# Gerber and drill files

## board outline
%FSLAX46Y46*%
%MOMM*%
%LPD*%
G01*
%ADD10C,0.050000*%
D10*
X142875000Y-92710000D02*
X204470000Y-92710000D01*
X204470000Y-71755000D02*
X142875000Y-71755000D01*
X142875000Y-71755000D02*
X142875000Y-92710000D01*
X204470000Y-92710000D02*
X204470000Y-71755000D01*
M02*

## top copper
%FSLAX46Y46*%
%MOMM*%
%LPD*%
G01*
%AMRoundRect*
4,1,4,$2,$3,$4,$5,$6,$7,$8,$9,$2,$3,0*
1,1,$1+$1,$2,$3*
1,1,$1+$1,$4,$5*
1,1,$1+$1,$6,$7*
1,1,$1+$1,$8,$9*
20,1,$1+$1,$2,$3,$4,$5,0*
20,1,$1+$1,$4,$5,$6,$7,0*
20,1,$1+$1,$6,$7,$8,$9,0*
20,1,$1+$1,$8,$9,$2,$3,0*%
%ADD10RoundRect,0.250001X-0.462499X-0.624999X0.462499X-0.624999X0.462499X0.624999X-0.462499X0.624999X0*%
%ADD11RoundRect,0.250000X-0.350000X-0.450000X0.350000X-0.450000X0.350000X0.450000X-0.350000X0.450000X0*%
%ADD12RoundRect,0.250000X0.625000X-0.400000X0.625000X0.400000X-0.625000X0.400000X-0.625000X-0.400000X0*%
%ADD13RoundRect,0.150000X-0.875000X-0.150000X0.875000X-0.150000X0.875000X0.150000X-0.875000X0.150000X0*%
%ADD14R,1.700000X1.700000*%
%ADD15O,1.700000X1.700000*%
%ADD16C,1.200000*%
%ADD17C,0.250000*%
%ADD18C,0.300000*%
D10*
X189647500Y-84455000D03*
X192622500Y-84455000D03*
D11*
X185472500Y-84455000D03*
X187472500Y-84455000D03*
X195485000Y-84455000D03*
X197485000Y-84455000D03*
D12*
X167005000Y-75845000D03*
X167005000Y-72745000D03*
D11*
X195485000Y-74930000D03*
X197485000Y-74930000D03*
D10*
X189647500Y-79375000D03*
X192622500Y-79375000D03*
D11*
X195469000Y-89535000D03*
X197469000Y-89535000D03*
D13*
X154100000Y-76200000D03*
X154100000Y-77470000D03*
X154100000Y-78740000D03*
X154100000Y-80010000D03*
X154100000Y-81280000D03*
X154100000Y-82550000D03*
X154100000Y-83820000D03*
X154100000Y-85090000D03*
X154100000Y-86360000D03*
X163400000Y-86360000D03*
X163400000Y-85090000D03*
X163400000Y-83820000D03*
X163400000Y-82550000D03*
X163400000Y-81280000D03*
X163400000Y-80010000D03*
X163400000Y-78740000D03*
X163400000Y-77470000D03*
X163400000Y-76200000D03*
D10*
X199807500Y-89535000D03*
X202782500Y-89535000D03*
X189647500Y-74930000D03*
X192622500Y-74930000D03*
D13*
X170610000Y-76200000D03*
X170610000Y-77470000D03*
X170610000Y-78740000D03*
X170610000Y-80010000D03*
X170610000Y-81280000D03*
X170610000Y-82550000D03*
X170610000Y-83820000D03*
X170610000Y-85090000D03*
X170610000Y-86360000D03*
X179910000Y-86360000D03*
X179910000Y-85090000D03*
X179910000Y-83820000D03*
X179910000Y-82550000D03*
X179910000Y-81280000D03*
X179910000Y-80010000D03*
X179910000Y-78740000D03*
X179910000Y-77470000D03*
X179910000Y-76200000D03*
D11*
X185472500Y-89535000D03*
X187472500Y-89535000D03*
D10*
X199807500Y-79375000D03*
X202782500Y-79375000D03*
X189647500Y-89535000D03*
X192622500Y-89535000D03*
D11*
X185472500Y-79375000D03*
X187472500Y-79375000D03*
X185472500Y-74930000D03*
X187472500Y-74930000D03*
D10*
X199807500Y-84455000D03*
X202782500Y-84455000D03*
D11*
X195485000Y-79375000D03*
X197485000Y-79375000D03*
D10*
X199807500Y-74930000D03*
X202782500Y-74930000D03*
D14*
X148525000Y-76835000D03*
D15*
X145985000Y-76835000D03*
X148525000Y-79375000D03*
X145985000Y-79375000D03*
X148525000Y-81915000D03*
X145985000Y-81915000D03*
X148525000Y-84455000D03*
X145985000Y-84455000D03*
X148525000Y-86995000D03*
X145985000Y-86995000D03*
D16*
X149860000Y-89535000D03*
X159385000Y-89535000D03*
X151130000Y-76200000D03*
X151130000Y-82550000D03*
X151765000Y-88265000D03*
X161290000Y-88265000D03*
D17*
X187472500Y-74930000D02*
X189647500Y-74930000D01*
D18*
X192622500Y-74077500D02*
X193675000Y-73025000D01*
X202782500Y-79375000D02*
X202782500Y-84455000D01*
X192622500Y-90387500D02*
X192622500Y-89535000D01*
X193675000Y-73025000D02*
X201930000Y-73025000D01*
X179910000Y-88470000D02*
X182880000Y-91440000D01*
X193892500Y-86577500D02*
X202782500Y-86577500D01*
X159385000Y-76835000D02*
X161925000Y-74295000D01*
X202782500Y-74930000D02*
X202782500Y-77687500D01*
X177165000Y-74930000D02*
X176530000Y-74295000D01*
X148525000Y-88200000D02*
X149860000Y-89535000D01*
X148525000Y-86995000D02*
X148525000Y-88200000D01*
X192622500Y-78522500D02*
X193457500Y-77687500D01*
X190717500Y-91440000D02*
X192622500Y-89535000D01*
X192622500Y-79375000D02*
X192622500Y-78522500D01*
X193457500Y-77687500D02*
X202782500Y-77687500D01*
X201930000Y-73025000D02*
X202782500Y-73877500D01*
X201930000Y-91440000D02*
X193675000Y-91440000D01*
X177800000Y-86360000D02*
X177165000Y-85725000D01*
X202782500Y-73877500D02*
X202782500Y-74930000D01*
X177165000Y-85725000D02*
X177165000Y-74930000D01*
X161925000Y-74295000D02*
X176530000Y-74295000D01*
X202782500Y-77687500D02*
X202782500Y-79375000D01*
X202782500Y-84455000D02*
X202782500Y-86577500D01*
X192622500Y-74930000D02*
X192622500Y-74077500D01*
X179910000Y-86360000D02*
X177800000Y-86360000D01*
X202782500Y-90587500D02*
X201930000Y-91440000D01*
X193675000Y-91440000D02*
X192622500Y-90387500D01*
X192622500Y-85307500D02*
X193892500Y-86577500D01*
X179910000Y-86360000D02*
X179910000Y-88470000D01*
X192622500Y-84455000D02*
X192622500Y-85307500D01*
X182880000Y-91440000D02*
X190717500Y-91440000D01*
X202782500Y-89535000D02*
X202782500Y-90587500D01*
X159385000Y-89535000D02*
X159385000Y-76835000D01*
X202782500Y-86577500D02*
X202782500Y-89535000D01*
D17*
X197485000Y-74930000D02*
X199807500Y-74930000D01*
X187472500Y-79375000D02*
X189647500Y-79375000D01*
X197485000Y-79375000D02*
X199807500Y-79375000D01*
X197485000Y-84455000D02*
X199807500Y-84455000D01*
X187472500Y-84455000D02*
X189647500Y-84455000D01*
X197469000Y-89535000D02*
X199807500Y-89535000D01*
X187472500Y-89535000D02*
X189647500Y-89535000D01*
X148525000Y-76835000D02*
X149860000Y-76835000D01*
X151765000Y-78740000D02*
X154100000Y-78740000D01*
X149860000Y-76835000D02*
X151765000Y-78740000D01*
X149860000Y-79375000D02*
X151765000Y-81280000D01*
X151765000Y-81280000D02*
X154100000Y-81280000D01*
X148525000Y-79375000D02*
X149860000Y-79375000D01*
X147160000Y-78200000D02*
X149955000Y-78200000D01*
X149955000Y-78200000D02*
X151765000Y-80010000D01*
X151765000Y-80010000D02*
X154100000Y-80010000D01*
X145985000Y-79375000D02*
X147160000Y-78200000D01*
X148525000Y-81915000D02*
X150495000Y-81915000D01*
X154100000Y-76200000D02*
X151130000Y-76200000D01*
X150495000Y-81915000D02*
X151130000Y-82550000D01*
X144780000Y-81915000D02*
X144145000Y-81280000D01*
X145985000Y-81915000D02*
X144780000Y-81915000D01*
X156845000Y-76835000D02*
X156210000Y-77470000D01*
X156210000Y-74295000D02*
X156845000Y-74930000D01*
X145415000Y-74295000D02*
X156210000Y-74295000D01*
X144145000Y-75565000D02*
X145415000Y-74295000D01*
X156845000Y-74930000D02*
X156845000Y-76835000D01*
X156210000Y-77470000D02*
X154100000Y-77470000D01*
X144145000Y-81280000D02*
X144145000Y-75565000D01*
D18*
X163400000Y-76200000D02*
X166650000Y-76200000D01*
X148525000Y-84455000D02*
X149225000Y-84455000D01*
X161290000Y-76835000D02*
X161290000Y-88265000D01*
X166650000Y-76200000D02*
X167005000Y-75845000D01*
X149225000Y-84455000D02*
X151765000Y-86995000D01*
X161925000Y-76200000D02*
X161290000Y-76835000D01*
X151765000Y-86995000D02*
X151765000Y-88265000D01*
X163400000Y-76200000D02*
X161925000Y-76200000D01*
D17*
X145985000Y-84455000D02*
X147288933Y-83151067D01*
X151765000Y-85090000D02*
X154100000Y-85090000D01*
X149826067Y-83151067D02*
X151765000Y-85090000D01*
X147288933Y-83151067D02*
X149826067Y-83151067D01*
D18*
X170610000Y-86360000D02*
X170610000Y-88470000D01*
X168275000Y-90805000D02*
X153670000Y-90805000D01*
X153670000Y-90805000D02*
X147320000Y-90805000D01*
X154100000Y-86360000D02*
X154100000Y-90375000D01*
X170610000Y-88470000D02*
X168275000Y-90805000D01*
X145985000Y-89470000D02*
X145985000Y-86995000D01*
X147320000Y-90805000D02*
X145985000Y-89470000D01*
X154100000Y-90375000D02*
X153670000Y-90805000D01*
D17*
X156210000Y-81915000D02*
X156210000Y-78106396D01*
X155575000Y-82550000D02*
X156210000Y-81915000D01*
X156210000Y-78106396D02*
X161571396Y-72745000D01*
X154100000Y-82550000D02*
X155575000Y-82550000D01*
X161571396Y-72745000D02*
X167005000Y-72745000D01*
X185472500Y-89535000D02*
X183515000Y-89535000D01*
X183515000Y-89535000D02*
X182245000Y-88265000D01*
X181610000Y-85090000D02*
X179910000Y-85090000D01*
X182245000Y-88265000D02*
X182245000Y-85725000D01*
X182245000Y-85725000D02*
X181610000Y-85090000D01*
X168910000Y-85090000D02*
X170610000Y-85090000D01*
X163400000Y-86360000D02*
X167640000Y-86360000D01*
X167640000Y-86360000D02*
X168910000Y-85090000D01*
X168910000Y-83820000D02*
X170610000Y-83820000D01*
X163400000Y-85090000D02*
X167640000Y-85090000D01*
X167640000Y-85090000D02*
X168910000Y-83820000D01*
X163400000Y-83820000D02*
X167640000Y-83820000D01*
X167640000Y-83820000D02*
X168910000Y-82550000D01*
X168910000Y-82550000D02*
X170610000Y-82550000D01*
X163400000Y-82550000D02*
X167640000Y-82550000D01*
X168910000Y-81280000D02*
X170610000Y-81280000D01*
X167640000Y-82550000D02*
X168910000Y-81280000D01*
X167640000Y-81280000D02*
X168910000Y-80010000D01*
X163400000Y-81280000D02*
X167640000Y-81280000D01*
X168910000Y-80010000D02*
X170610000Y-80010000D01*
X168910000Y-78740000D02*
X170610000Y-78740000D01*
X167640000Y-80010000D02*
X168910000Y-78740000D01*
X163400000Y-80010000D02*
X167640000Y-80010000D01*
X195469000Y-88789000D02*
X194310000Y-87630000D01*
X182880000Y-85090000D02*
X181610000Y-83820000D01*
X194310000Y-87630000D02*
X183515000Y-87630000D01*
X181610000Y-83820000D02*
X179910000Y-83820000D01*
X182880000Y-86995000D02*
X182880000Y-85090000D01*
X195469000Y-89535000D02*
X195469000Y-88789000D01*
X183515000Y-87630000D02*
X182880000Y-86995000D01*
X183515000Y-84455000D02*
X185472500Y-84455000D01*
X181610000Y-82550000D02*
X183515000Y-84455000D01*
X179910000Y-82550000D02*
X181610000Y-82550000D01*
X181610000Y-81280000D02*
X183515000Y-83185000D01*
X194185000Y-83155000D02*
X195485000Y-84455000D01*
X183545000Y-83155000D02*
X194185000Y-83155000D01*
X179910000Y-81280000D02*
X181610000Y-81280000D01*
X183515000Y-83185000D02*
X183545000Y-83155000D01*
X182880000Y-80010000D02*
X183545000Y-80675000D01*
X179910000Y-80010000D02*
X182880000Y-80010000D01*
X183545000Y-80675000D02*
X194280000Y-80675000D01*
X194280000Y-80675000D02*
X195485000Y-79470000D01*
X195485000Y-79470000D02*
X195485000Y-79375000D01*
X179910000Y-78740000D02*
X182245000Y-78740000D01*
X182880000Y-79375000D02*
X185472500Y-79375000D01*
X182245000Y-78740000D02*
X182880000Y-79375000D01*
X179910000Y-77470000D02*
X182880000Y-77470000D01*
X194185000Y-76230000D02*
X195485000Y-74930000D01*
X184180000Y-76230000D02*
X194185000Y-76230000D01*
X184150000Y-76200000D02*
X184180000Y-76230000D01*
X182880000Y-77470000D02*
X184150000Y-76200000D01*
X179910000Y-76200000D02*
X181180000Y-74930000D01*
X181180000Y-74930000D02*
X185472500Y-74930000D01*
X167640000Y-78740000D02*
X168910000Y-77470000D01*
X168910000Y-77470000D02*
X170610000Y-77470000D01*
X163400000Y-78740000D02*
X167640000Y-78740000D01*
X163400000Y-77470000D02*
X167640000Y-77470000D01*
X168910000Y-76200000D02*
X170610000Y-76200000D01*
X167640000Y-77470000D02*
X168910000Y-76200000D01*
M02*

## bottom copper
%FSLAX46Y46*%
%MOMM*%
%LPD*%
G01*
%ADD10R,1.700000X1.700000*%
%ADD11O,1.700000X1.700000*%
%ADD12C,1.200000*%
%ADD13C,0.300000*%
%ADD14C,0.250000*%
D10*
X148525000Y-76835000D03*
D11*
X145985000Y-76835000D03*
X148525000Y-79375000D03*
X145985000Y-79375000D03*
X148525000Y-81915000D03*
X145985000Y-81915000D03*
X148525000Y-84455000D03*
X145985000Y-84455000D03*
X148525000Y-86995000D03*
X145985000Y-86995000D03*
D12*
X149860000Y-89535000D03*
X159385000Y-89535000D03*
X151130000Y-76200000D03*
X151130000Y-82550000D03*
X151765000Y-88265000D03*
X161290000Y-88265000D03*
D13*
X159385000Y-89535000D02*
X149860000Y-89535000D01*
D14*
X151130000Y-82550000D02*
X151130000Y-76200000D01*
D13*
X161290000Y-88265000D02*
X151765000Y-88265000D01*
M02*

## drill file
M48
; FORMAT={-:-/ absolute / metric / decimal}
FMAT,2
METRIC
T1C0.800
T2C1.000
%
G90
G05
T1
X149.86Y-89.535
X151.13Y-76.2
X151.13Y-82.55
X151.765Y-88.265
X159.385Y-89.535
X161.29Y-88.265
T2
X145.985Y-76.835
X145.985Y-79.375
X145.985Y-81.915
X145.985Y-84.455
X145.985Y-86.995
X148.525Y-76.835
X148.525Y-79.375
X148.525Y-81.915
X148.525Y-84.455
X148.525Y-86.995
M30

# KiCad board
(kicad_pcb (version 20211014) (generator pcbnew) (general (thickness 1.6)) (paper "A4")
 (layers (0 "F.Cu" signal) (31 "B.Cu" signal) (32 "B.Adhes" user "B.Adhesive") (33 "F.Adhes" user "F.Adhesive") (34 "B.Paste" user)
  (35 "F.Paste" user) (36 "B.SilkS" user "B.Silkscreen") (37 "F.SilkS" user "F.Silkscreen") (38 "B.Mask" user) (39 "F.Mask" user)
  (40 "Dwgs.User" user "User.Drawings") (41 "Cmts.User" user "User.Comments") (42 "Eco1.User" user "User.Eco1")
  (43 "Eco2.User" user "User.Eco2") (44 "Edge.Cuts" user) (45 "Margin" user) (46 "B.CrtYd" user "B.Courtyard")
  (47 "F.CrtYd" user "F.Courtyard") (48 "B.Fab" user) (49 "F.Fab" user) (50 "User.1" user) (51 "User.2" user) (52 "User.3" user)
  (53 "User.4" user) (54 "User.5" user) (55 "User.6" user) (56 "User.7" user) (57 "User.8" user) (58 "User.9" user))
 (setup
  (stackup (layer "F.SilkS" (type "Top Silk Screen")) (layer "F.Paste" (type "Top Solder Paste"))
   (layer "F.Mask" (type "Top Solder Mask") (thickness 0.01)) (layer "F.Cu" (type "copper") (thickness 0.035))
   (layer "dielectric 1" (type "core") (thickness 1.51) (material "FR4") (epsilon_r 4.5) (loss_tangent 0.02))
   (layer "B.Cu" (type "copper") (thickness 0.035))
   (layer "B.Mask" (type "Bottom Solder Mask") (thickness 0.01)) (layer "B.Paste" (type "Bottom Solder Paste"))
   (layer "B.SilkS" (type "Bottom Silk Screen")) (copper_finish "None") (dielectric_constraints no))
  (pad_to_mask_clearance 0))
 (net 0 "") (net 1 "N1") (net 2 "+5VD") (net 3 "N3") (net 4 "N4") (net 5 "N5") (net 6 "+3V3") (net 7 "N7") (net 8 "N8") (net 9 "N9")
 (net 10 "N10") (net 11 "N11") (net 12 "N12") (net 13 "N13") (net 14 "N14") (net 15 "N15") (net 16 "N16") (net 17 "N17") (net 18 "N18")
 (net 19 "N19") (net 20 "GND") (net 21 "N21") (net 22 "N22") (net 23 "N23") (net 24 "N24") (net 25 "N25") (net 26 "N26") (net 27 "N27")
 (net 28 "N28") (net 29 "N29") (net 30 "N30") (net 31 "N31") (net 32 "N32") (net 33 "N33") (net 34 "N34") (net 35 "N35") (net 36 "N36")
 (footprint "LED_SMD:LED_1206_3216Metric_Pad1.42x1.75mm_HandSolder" (layer "F.Cu") (at 191.135 84.455)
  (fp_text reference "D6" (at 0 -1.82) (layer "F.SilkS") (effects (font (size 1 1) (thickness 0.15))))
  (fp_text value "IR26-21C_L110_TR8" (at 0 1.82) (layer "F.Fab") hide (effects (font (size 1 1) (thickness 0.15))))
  (pad "1" smd roundrect (at -1.4875 0) (size 1.425 1.75) (layers "F.Cu" "F.Paste" "F.Mask") (roundrect_rratio 0.175439) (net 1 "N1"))
  (pad "2" smd roundrect (at 1.4875 0) (size 1.425 1.75) (layers "F.Cu" "F.Paste" "F.Mask") (roundrect_rratio 0.175439) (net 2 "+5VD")))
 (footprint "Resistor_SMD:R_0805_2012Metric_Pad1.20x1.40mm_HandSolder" (layer "F.Cu") (at 186.4725 84.455)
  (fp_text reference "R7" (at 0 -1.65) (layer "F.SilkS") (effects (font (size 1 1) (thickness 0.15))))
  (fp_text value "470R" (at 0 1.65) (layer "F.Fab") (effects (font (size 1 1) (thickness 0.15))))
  (pad "1" smd roundrect (at -1 0) (size 1.2 1.4) (layers "F.Cu" "F.Paste" "F.Mask") (roundrect_rratio 0.208333) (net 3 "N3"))
  (pad "2" smd roundrect (at 1 0) (size 1.2 1.4) (layers "F.Cu" "F.Paste" "F.Mask") (roundrect_rratio 0.208333) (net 1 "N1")))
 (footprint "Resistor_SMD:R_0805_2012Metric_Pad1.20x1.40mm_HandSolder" (layer "F.Cu") (at 196.485 84.455)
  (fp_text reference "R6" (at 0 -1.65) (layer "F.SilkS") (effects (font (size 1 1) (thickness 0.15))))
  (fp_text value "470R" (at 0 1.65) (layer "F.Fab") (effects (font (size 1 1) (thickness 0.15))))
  (pad "1" smd roundrect (at -1 0) (size 1.2 1.4) (layers "F.Cu" "F.Paste" "F.Mask") (roundrect_rratio 0.208333) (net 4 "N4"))
  (pad "2" smd roundrect (at 1 0) (size 1.2 1.4) (layers "F.Cu" "F.Paste" "F.Mask") (roundrect_rratio 0.208333) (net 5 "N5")))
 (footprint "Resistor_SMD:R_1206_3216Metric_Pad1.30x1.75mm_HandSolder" (layer "F.Cu") (at 167.005 74.295 90)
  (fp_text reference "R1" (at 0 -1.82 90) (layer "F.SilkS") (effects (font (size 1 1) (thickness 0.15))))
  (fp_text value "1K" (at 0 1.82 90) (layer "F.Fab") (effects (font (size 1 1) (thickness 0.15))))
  (pad "1" smd roundrect (at -1.55 0 90) (size 1.3 1.75) (layers "F.Cu" "F.Paste" "F.Mask") (roundrect_rratio 0.192308) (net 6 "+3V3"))
  (pad "2" smd roundrect (at 1.55 0 90) (size 1.3 1.75) (layers "F.Cu" "F.Paste" "F.Mask") (roundrect_rratio 0.192308) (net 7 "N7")))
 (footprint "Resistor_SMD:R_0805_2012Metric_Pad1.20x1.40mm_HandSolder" (layer "F.Cu") (at 196.485 74.93)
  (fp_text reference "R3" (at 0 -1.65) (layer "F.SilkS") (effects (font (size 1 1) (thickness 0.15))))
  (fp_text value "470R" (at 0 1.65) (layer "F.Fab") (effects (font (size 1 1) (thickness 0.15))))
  (pad "1" smd roundrect (at -1 0) (size 1.2 1.4) (layers "F.Cu" "F.Paste" "F.Mask") (roundrect_rratio 0.208333) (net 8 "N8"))
  (pad "2" smd roundrect (at 1 0) (size 1.2 1.4) (layers "F.Cu" "F.Paste" "F.Mask") (roundrect_rratio 0.208333) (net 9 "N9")))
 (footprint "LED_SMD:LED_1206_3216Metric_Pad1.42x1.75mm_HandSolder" (layer "F.Cu") (at 191.135 79.375)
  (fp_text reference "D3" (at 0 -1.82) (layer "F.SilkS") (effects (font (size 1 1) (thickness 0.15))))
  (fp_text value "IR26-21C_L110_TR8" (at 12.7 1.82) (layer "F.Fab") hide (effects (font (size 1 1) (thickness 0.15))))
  (pad "1" smd roundrect (at -1.4875 0) (size 1.425 1.75) (layers "F.Cu" "F.Paste" "F.Mask") (roundrect_rratio 0.175439) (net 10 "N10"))
  (pad "2" smd roundrect (at 1.4875 0) (size 1.425 1.75) (layers "F.Cu" "F.Paste" "F.Mask") (roundrect_rratio 0.175439) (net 2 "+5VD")))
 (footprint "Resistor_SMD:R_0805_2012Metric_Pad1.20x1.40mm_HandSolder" (layer "F.Cu") (at 196.469 89.535)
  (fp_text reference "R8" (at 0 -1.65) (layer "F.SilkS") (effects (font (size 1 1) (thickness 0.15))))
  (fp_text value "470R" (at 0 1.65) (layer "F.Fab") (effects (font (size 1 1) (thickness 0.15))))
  (pad "1" smd roundrect (at -1 0) (size 1.2 1.4) (layers "F.Cu" "F.Paste" "F.Mask") (roundrect_rratio 0.208333) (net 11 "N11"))
  (pad "2" smd roundrect (at 1 0) (size 1.2 1.4) (layers "F.Cu" "F.Paste" "F.Mask") (roundrect_rratio 0.208333) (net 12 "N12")))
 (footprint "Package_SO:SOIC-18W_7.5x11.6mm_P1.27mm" (layer "F.Cu") (at 158.75 81.28)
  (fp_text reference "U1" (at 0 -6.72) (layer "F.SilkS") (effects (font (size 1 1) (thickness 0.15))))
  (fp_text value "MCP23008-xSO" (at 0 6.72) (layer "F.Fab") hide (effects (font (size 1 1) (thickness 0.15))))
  (pad "1" smd roundrect (at -4.65 -5.08) (size 2.05 0.6) (layers "F.Cu" "F.Paste" "F.Mask") (roundrect_rratio 0.25) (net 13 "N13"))
  (pad "2" smd roundrect (at -4.65 -3.81) (size 2.05 0.6) (layers "F.Cu" "F.Paste" "F.Mask") (roundrect_rratio 0.25) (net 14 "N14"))
  (pad "3" smd roundrect (at -4.65 -2.54) (size 2.05 0.6) (layers "F.Cu" "F.Paste" "F.Mask") (roundrect_rratio 0.25) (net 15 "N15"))
  (pad "4" smd roundrect (at -4.65 -1.27) (size 2.05 0.6) (layers "F.Cu" "F.Paste" "F.Mask") (roundrect_rratio 0.25) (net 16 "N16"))
  (pad "5" smd roundrect (at -4.65 0) (size 2.05 0.6) (layers "F.Cu" "F.Paste" "F.Mask") (roundrect_rratio 0.25) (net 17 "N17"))
  (pad "6" smd roundrect (at -4.65 1.27) (size 2.05 0.6) (layers "F.Cu" "F.Paste" "F.Mask") (roundrect_rratio 0.25) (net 7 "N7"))
  (pad "7" smd roundrect (at -4.65 2.54) (size 2.05 0.6) (layers "F.Cu" "F.Paste" "F.Mask") (roundrect_rratio 0.25) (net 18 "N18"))
  (pad "8" smd roundrect (at -4.65 3.81) (size 2.05 0.6) (layers "F.Cu" "F.Paste" "F.Mask") (roundrect_rratio 0.25) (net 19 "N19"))
  (pad "9" smd roundrect (at -4.65 5.08) (size 2.05 0.6) (layers "F.Cu" "F.Paste" "F.Mask") (roundrect_rratio 0.25) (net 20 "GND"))
  (pad "10" smd roundrect (at 4.65 5.08) (size 2.05 0.6) (layers "F.Cu" "F.Paste" "F.Mask") (roundrect_rratio 0.25) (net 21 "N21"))
  (pad "11" smd roundrect (at 4.65 3.81) (size 2.05 0.6) (layers "F.Cu" "F.Paste" "F.Mask") (roundrect_rratio 0.25) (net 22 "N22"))
  (pad "12" smd roundrect (at 4.65 2.54) (size 2.05 0.6) (layers "F.Cu" "F.Paste" "F.Mask") (roundrect_rratio 0.25) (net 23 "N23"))
  (pad "13" smd roundrect (at 4.65 1.27) (size 2.05 0.6) (layers "F.Cu" "F.Paste" "F.Mask") (roundrect_rratio 0.25) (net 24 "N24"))
  (pad "14" smd roundrect (at 4.65 0) (size 2.05 0.6) (layers "F.Cu" "F.Paste" "F.Mask") (roundrect_rratio 0.25) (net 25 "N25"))
  (pad "15" smd roundrect (at 4.65 -1.27) (size 2.05 0.6) (layers "F.Cu" "F.Paste" "F.Mask") (roundrect_rratio 0.25) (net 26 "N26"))
  (pad "16" smd roundrect (at 4.65 -2.54) (size 2.05 0.6) (layers "F.Cu" "F.Paste" "F.Mask") (roundrect_rratio 0.25) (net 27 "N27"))
  (pad "17" smd roundrect (at 4.65 -3.81) (size 2.05 0.6) (layers "F.Cu" "F.Paste" "F.Mask") (roundrect_rratio 0.25) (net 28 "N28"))
  (pad "18" smd roundrect (at 4.65 -5.08) (size 2.05 0.6) (layers "F.Cu" "F.Paste" "F.Mask") (roundrect_rratio 0.25) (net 6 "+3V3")))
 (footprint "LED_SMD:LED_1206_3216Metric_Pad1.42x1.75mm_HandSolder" (layer "F.Cu") (at 201.295 89.535)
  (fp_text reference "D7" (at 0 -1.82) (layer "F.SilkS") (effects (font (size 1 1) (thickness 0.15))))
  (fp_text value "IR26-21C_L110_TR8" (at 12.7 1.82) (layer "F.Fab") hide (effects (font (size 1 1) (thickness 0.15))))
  (pad "1" smd roundrect (at -1.4875 0) (size 1.425 1.75) (layers "F.Cu" "F.Paste" "F.Mask") (roundrect_rratio 0.175439) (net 12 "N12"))
  (pad "2" smd roundrect (at 1.4875 0) (size 1.425 1.75) (layers "F.Cu" "F.Paste" "F.Mask") (roundrect_rratio 0.175439) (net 2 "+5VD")))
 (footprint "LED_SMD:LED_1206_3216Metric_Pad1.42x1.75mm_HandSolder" (layer "F.Cu") (at 191.135 74.93)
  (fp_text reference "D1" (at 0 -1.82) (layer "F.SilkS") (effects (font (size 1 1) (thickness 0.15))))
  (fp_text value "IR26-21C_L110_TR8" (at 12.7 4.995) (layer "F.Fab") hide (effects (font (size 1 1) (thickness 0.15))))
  (pad "1" smd roundrect (at -1.4875 0) (size 1.425 1.75) (layers "F.Cu" "F.Paste" "F.Mask") (roundrect_rratio 0.175439) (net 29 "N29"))
  (pad "2" smd roundrect (at 1.4875 0) (size 1.425 1.75) (layers "F.Cu" "F.Paste" "F.Mask") (roundrect_rratio 0.175439) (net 2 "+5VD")))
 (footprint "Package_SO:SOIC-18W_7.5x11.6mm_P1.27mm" (layer "F.Cu") (at 175.26 81.28)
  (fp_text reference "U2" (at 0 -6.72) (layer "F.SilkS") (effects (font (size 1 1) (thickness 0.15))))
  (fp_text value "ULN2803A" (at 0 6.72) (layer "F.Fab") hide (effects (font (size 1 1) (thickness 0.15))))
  (pad "1" smd roundrect (at -4.65 -5.08) (size 2.05 0.6) (layers "F.Cu" "F.Paste" "F.Mask") (roundrect_rratio 0.25) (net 28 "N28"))
  (pad "2" smd roundrect (at -4.65 -3.81) (size 2.05 0.6) (layers "F.Cu" "F.Paste" "F.Mask") (roundrect_rratio 0.25) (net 27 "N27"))
  (pad "3" smd roundrect (at -4.65 -2.54) (size 2.05 0.6) (layers "F.Cu" "F.Paste" "F.Mask") (roundrect_rratio 0.25) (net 26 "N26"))
  (pad "4" smd roundrect (at -4.65 -1.27) (size 2.05 0.6) (layers "F.Cu" "F.Paste" "F.Mask") (roundrect_rratio 0.25) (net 25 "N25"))
  (pad "5" smd roundrect (at -4.65 0) (size 2.05 0.6) (layers "F.Cu" "F.Paste" "F.Mask") (roundrect_rratio 0.25) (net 24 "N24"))
  (pad "6" smd roundrect (at -4.65 1.27) (size 2.05 0.6) (layers "F.Cu" "F.Paste" "F.Mask") (roundrect_rratio 0.25) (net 23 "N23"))
  (pad "7" smd roundrect (at -4.65 2.54) (size 2.05 0.6) (layers "F.Cu" "F.Paste" "F.Mask") (roundrect_rratio 0.25) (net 22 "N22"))
  (pad "8" smd roundrect (at -4.65 3.81) (size 2.05 0.6) (layers "F.Cu" "F.Paste" "F.Mask") (roundrect_rratio 0.25) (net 21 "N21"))
  (pad "9" smd roundrect (at -4.65 5.08) (size 2.05 0.6) (layers "F.Cu" "F.Paste" "F.Mask") (roundrect_rratio 0.25) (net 20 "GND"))
  (pad "10" smd roundrect (at 4.65 5.08) (size 2.05 0.6) (layers "F.Cu" "F.Paste" "F.Mask") (roundrect_rratio 0.25) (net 2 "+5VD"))
  (pad "11" smd roundrect (at 4.65 3.81) (size 2.05 0.6) (layers "F.Cu" "F.Paste" "F.Mask") (roundrect_rratio 0.25) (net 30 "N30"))
  (pad "12" smd roundrect (at 4.65 2.54) (size 2.05 0.6) (layers "F.Cu" "F.Paste" "F.Mask") (roundrect_rratio 0.25) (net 11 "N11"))
  (pad "13" smd roundrect (at 4.65 1.27) (size 2.05 0.6) (layers "F.Cu" "F.Paste" "F.Mask") (roundrect_rratio 0.25) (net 3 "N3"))
  (pad "14" smd roundrect (at 4.65 0) (size 2.05 0.6) (layers "F.Cu" "F.Paste" "F.Mask") (roundrect_rratio 0.25) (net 4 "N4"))
  (pad "15" smd roundrect (at 4.65 -1.27) (size 2.05 0.6) (layers "F.Cu" "F.Paste" "F.Mask") (roundrect_rratio 0.25) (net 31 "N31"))
  (pad "16" smd roundrect (at 4.65 -2.54) (size 2.05 0.6) (layers "F.Cu" "F.Paste" "F.Mask") (roundrect_rratio 0.25) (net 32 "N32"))
  (pad "17" smd roundrect (at 4.65 -3.81) (size 2.05 0.6) (layers "F.Cu" "F.Paste" "F.Mask") (roundrect_rratio 0.25) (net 8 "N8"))
  (pad "18" smd roundrect (at 4.65 -5.08) (size 2.05 0.6) (layers "F.Cu" "F.Paste" "F.Mask") (roundrect_rratio 0.25) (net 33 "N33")))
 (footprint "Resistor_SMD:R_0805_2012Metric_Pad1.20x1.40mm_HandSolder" (layer "F.Cu") (at 186.4725 89.535)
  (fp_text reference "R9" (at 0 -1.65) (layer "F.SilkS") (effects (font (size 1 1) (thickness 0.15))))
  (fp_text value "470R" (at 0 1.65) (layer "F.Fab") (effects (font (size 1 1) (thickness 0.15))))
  (pad "1" smd roundrect (at -1 0) (size 1.2 1.4) (layers "F.Cu" "F.Paste" "F.Mask") (roundrect_rratio 0.208333) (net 30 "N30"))
  (pad "2" smd roundrect (at 1 0) (size 1.2 1.4) (layers "F.Cu" "F.Paste" "F.Mask") (roundrect_rratio 0.208333) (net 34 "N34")))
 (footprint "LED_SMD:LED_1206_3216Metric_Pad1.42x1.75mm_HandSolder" (layer "F.Cu") (at 201.295 79.375)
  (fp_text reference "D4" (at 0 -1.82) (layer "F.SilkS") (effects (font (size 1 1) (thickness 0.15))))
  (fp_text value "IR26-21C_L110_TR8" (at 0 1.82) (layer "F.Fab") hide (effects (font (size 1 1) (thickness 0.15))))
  (pad "1" smd roundrect (at -1.4875 0) (size 1.425 1.75) (layers "F.Cu" "F.Paste" "F.Mask") (roundrect_rratio 0.175439) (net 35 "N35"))
  (pad "2" smd roundrect (at 1.4875 0) (size 1.425 1.75) (layers "F.Cu" "F.Paste" "F.Mask") (roundrect_rratio 0.175439) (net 2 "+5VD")))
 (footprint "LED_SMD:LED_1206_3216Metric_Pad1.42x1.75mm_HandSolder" (layer "F.Cu") (at 191.135 89.535)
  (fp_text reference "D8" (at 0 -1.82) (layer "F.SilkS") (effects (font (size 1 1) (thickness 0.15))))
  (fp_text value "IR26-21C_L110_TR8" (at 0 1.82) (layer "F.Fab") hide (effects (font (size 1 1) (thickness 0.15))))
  (pad "1" smd roundrect (at -1.4875 0) (size 1.425 1.75) (layers "F.Cu" "F.Paste" "F.Mask") (roundrect_rratio 0.175439) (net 34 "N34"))
  (pad "2" smd roundrect (at 1.4875 0) (size 1.425 1.75) (layers "F.Cu" "F.Paste" "F.Mask") (roundrect_rratio 0.175439) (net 2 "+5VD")))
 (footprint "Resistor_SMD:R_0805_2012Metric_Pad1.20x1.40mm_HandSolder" (layer "F.Cu") (at 186.4725 79.375)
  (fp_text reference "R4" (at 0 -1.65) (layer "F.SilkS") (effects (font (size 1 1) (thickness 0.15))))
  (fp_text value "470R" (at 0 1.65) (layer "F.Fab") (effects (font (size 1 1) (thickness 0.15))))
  (pad "1" smd roundrect (at -1 0) (size 1.2 1.4) (layers "F.Cu" "F.Paste" "F.Mask") (roundrect_rratio 0.208333) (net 32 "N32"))
  (pad "2" smd roundrect (at 1 0) (size 1.2 1.4) (layers "F.Cu" "F.Paste" "F.Mask") (roundrect_rratio 0.208333) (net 10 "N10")))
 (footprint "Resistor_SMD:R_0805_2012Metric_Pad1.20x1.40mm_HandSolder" (layer "F.Cu") (at 186.4725 74.93)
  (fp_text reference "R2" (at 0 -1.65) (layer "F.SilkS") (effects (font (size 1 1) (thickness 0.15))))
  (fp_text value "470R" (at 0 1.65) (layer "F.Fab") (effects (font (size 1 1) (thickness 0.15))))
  (pad "1" smd roundrect (at -1 0) (size 1.2 1.4) (layers "F.Cu" "F.Paste" "F.Mask") (roundrect_rratio 0.208333) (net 33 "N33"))
  (pad "2" smd roundrect (at 1 0) (size 1.2 1.4) (layers "F.Cu" "F.Paste" "F.Mask") (roundrect_rratio 0.208333) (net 29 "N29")))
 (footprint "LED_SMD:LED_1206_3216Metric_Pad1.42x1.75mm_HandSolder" (layer "F.Cu") (at 201.295 84.455)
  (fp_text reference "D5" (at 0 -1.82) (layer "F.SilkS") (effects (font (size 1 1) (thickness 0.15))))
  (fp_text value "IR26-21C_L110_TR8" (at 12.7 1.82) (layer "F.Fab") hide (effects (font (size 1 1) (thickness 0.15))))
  (pad "1" smd roundrect (at -1.4875 0) (size 1.425 1.75) (layers "F.Cu" "F.Paste" "F.Mask") (roundrect_rratio 0.175439) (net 5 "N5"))
  (pad "2" smd roundrect (at 1.4875 0) (size 1.425 1.75) (layers "F.Cu" "F.Paste" "F.Mask") (roundrect_rratio 0.175439) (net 2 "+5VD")))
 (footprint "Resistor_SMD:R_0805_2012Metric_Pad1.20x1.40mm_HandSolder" (layer "F.Cu") (at 196.485 79.375)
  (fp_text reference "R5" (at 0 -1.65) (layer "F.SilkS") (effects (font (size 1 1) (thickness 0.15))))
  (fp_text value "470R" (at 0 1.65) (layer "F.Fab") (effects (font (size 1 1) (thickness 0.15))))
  (pad "1" smd roundrect (at -1 0) (size 1.2 1.4) (layers "F.Cu" "F.Paste" "F.Mask") (roundrect_rratio 0.208333) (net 31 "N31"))
  (pad "2" smd roundrect (at 1 0) (size 1.2 1.4) (layers "F.Cu" "F.Paste" "F.Mask") (roundrect_rratio 0.208333) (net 35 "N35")))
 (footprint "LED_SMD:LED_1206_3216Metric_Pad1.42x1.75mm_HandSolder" (layer "F.Cu") (at 201.295 74.93)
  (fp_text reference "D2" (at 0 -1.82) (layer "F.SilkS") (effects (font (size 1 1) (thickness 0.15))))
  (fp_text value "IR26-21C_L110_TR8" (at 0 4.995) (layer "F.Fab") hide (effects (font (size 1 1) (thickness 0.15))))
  (pad "1" smd roundrect (at -1.4875 0) (size 1.425 1.75) (layers "F.Cu" "F.Paste" "F.Mask") (roundrect_rratio 0.175439) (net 9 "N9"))
  (pad "2" smd roundrect (at 1.4875 0) (size 1.425 1.75) (layers "F.Cu" "F.Paste" "F.Mask") (roundrect_rratio 0.175439) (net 2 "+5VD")))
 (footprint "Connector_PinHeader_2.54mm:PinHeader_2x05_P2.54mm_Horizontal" (layer "B.Cu") (at 148.525 76.835 180)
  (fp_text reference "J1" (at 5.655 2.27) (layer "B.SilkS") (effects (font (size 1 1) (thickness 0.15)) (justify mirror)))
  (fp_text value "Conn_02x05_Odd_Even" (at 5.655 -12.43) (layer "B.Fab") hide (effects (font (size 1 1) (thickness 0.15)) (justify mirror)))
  (pad "1" thru_hole rect (at 0 0 180) (size 1.7 1.7) (drill 1) (layers *.Cu *.Mask) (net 15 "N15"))
  (pad "2" thru_hole oval (at 2.54 0 180) (size 1.7 1.7) (drill 1) (layers *.Cu *.Mask) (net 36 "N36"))
  (pad "3" thru_hole oval (at 0 -2.54 180) (size 1.7 1.7) (drill 1) (layers *.Cu *.Mask) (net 17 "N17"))
  (pad "4" thru_hole oval (at 2.54 -2.54 180) (size 1.7 1.7) (drill 1) (layers *.Cu *.Mask) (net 16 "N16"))
  (pad "5" thru_hole oval (at 0 -5.08 180) (size 1.7 1.7) (drill 1) (layers *.Cu *.Mask) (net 13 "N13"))
  (pad "6" thru_hole oval (at 2.54 -5.08 180) (size 1.7 1.7) (drill 1) (layers *.Cu *.Mask) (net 14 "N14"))
  (pad "7" thru_hole oval (at 0 -7.62 180) (size 1.7 1.7) (drill 1) (layers *.Cu *.Mask) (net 6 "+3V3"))
  (pad "8" thru_hole oval (at 2.54 -7.62 180) (size 1.7 1.7) (drill 1) (layers *.Cu *.Mask) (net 19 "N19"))
  (pad "9" thru_hole oval (at 0 -10.16 180) (size 1.7 1.7) (drill 1) (layers *.Cu *.Mask) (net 2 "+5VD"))
  (pad "10" thru_hole oval (at 2.54 -10.16 180) (size 1.7 1.7) (drill 1) (layers *.Cu *.Mask) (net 20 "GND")))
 (gr_line (start 142.875 92.71) (end 204.47 92.71) (layer "Edge.Cuts") (width 0.05))
 (gr_line (start 204.47 71.755) (end 142.875 71.755) (layer "Edge.Cuts") (width 0.05))
 (gr_line (start 142.875 71.755) (end 142.875 92.71) (layer "Edge.Cuts") (width 0.05))
 (gr_line (start 204.47 92.71) (end 204.47 71.755) (layer "Edge.Cuts") (width 0.05))
 (segment (start 187.4725 74.93) (end 189.6475 74.93) (width 0.25) (layer "F.Cu") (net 29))
 (segment (start 192.6225 74.0775) (end 193.675 73.025) (width 0.3) (layer "F.Cu") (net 2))
 (segment (start 202.7825 79.375) (end 202.7825 84.455) (width 0.3) (layer "F.Cu") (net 2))
 (segment (start 192.6225 90.3875) (end 192.6225 89.535) (width 0.3) (layer "F.Cu") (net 2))
 (segment (start 193.675 73.025) (end 201.93 73.025) (width 0.3) (layer "F.Cu") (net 2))
 (segment (start 179.91 88.47) (end 182.88 91.44) (width 0.3) (layer "F.Cu") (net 2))
 (segment (start 193.8925 86.5775) (end 202.7825 86.5775) (width 0.3) (layer "F.Cu") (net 2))
 (segment (start 159.385 76.835) (end 161.925 74.295) (width 0.3) (layer "F.Cu") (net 2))
 (segment (start 202.7825 74.93) (end 202.7825 77.6875) (width 0.3) (layer "F.Cu") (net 2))
 (segment (start 177.165 74.93) (end 176.53 74.295) (width 0.3) (layer "F.Cu") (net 2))
 (segment (start 148.525 88.2) (end 149.86 89.535) (width 0.3) (layer "F.Cu") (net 2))
 (segment (start 148.525 86.995) (end 148.525 88.2) (width 0.3) (layer "F.Cu") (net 2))
 (segment (start 192.6225 78.5225) (end 193.4575 77.6875) (width 0.3) (layer "F.Cu") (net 2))
 (segment (start 190.7175 91.44) (end 192.6225 89.535) (width 0.3) (layer "F.Cu") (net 2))
 (segment (start 192.6225 79.375) (end 192.6225 78.5225) (width 0.3) (layer "F.Cu") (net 2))
 (segment (start 193.4575 77.6875) (end 202.7825 77.6875) (width 0.3) (layer "F.Cu") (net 2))
 (segment (start 201.93 73.025) (end 202.7825 73.8775) (width 0.3) (layer "F.Cu") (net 2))
 (segment (start 201.93 91.44) (end 193.675 91.44) (width 0.3) (layer "F.Cu") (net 2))
 (segment (start 177.8 86.36) (end 177.165 85.725) (width 0.3) (layer "F.Cu") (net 2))
 (segment (start 202.7825 73.8775) (end 202.7825 74.93) (width 0.3) (layer "F.Cu") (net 2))
 (segment (start 177.165 85.725) (end 177.165 74.93) (width 0.3) (layer "F.Cu") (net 2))
 (segment (start 161.925 74.295) (end 176.53 74.295) (width 0.3) (layer "F.Cu") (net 2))
 (segment (start 202.7825 77.6875) (end 202.7825 79.375) (width 0.3) (layer "F.Cu") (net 2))
 (segment (start 202.7825 84.455) (end 202.7825 86.5775) (width 0.3) (layer "F.Cu") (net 2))
 (segment (start 192.6225 74.93) (end 192.6225 74.0775) (width 0.3) (layer "F.Cu") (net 2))
 (segment (start 179.91 86.36) (end 177.8 86.36) (width 0.3) (layer "F.Cu") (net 2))
 (segment (start 202.7825 90.5875) (end 201.93 91.44) (width 0.3) (layer "F.Cu") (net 2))
 (segment (start 193.675 91.44) (end 192.6225 90.3875) (width 0.3) (layer "F.Cu") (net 2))
 (segment (start 192.6225 85.3075) (end 193.8925 86.5775) (width 0.3) (layer "F.Cu") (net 2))
 (segment (start 179.91 86.36) (end 179.91 88.47) (width 0.3) (layer "F.Cu") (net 2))
 (segment (start 192.6225 84.455) (end 192.6225 85.3075) (width 0.3) (layer "F.Cu") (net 2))
 (segment (start 182.88 91.44) (end 190.7175 91.44) (width 0.3) (layer "F.Cu") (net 2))
 (segment (start 202.7825 89.535) (end 202.7825 90.5875) (width 0.3) (layer "F.Cu") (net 2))
 (segment (start 159.385 89.535) (end 159.385 76.835) (width 0.3) (layer "F.Cu") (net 2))
 (segment (start 202.7825 86.5775) (end 202.7825 89.535) (width 0.3) (layer "F.Cu") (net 2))
 (via (at 149.86 89.535) (size 1.2) (drill 0.8) (layers "F.Cu" "B.Cu") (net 2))
 (via (at 159.385 89.535) (size 1.2) (drill 0.8) (layers "F.Cu" "B.Cu") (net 2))
 (segment (start 159.385 89.535) (end 149.86 89.535) (width 0.3) (layer "B.Cu") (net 2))
 (segment (start 197.485 74.93) (end 199.8075 74.93) (width 0.25) (layer "F.Cu") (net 9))
 (segment (start 187.4725 79.375) (end 189.6475 79.375) (width 0.25) (layer "F.Cu") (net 10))
 (segment (start 197.485 79.375) (end 199.8075 79.375) (width 0.25) (layer "F.Cu") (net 35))
 (segment (start 197.485 84.455) (end 199.8075 84.455) (width 0.25) (layer "F.Cu") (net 5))
 (segment (start 187.4725 84.455) (end 189.6475 84.455) (width 0.25) (layer "F.Cu") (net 1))
 (segment (start 197.469 89.535) (end 199.8075 89.535) (width 0.25) (layer "F.Cu") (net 12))
 (segment (start 187.4725 89.535) (end 189.6475 89.535) (width 0.25) (layer "F.Cu") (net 34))
 (segment (start 148.525 76.835) (end 149.86 76.835) (width 0.25) (layer "F.Cu") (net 15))
 (segment (start 151.765 78.74) (end 154.1 78.74) (width 0.25) (layer "F.Cu") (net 15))
 (segment (start 149.86 76.835) (end 151.765 78.74) (width 0.25) (layer "F.Cu") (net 15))
 (segment (start 149.86 79.375) (end 151.765 81.28) (width 0.25) (layer "F.Cu") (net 17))
 (segment (start 151.765 81.28) (end 154.1 81.28) (width 0.25) (layer "F.Cu") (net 17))
 (segment (start 148.525 79.375) (end 149.86 79.375) (width 0.25) (layer "F.Cu") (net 17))
 (segment (start 147.16 78.2) (end 149.955 78.2) (width 0.25) (layer "F.Cu") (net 16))
 (segment (start 149.955 78.2) (end 151.765 80.01) (width 0.25) (layer "F.Cu") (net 16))
 (segment (start 151.765 80.01) (end 154.1 80.01) (width 0.25) (layer "F.Cu") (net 16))
 (segment (start 145.985 79.375) (end 147.16 78.2) (width 0.25) (layer "F.Cu") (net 16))
 (segment (start 148.525 81.915) (end 150.495 81.915) (width 0.25) (layer "F.Cu") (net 13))
 (segment (start 154.1 76.2) (end 151.13 76.2) (width 0.25) (layer "F.Cu") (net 13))
 (segment (start 150.495 81.915) (end 151.13 82.55) (width 0.25) (layer "F.Cu") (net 13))
 (via (at 151.13 76.2) (size 1.2) (drill 0.8) (layers "F.Cu" "B.Cu") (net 13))
 (via (at 151.13 82.55) (size 1.2) (drill 0.8) (layers "F.Cu" "B.Cu") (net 13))
 (segment (start 151.13 82.55) (end 151.13 76.2) (width 0.25) (layer "B.Cu") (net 13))
 (segment (start 144.78 81.915) (end 144.145 81.28) (width 0.25) (layer "F.Cu") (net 14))
 (segment (start 145.985 81.915) (end 144.78 81.915) (width 0.25) (layer "F.Cu") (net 14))
 (segment (start 156.845 76.835) (end 156.21 77.47) (width 0.25) (layer "F.Cu") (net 14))
 (segment (start 156.21 74.295) (end 156.845 74.93) (width 0.25) (layer "F.Cu") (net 14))
 (segment (start 145.415 74.295) (end 156.21 74.295) (width 0.25) (layer "F.Cu") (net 14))
 (segment (start 144.145 75.565) (end 145.415 74.295) (width 0.25) (layer "F.Cu") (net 14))
 (segment (start 156.845 74.93) (end 156.845 76.835) (width 0.25) (layer "F.Cu") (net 14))
 (segment (start 156.21 77.47) (end 154.1 77.47) (width 0.25) (layer "F.Cu") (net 14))
 (segment (start 144.145 81.28) (end 144.145 75.565) (width 0.25) (layer "F.Cu") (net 14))
 (segment (start 163.4 76.2) (end 166.65 76.2) (width 0.3) (layer "F.Cu") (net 6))
 (segment (start 148.525 84.455) (end 149.225 84.455) (width 0.3) (layer "F.Cu") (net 6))
 (segment (start 161.29 76.835) (end 161.29 88.265) (width 0.3) (layer "F.Cu") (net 6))
 (segment (start 166.65 76.2) (end 167.005 75.845) (width 0.3) (layer "F.Cu") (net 6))
 (segment (start 149.225 84.455) (end 151.765 86.995) (width 0.3) (layer "F.Cu") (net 6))
 (segment (start 161.925 76.2) (end 161.29 76.835) (width 0.3) (layer "F.Cu") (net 6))
 (segment (start 151.765 86.995) (end 151.765 88.265) (width 0.3) (layer "F.Cu") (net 6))
 (segment (start 163.4 76.2) (end 161.925 76.2) (width 0.3) (layer "F.Cu") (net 6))
 (via (at 151.765 88.265) (size 1.2) (drill 0.8) (layers "F.Cu" "B.Cu") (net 6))
 (via (at 161.29 88.265) (size 1.2) (drill 0.8) (layers "F.Cu" "B.Cu") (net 6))
 (segment (start 161.29 88.265) (end 151.765 88.265) (width 0.3) (layer "B.Cu") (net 6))
 (segment (start 145.985 84.455) (end 147.288933 83.151067) (width 0.25) (layer "F.Cu") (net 19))
 (segment (start 151.765 85.09) (end 154.1 85.09) (width 0.25) (layer "F.Cu") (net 19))
 (segment (start 149.826067 83.151067) (end 151.765 85.09) (width 0.25) (layer "F.Cu") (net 19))
 (segment (start 147.288933 83.151067) (end 149.826067 83.151067) (width 0.25) (layer "F.Cu") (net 19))
 (segment (start 170.61 86.36) (end 170.61 88.47) (width 0.3) (layer "F.Cu") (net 20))
 (segment (start 168.275 90.805) (end 153.67 90.805) (width 0.3) (layer "F.Cu") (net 20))
 (segment (start 153.67 90.805) (end 147.32 90.805) (width 0.3) (layer "F.Cu") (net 20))
 (segment (start 154.1 86.36) (end 154.1 90.375) (width 0.3) (layer "F.Cu") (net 20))
 (segment (start 170.61 88.47) (end 168.275 90.805) (width 0.3) (layer "F.Cu") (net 20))
 (segment (start 145.985 89.47) (end 145.985 86.995) (width 0.3) (layer "F.Cu") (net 20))
 (segment (start 147.32 90.805) (end 145.985 89.47) (width 0.3) (layer "F.Cu") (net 20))
 (segment (start 154.1 90.375) (end 153.67 90.805) (width 0.3) (layer "F.Cu") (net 20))
 (segment (start 156.21 81.915) (end 156.21 78.106396) (width 0.25) (layer "F.Cu") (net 7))
 (segment (start 155.575 82.55) (end 156.21 81.915) (width 0.25) (layer "F.Cu") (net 7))
 (segment (start 156.21 78.106396) (end 161.571396 72.745) (width 0.25) (layer "F.Cu") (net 7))
 (segment (start 154.1 82.55) (end 155.575 82.55) (width 0.25) (layer "F.Cu") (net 7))
 (segment (start 161.571396 72.745) (end 167.005 72.745) (width 0.25) (layer "F.Cu") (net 7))
 (segment (start 185.4725 89.535) (end 183.515 89.535) (width 0.25) (layer "F.Cu") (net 30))
 (segment (start 183.515 89.535) (end 182.245 88.265) (width 0.25) (layer "F.Cu") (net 30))
 (segment (start 181.61 85.09) (end 179.91 85.09) (width 0.25) (layer "F.Cu") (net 30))
 (segment (start 182.245 88.265) (end 182.245 85.725) (width 0.25) (layer "F.Cu") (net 30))
 (segment (start 182.245 85.725) (end 181.61 85.09) (width 0.25) (layer "F.Cu") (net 30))
 (segment (start 168.91 85.09) (end 170.61 85.09) (width 0.25) (layer "F.Cu") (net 21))
 (segment (start 163.4 86.36) (end 167.64 86.36) (width 0.25) (layer "F.Cu") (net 21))
 (segment (start 167.64 86.36) (end 168.91 85.09) (width 0.25) (layer "F.Cu") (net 21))
 (segment (start 168.91 83.82) (end 170.61 83.82) (width 0.25) (layer "F.Cu") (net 22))
 (segment (start 163.4 85.09) (end 167.64 85.09) (width 0.25) (layer "F.Cu") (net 22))
 (segment (start 167.64 85.09) (end 168.91 83.82) (width 0.25) (layer "F.Cu") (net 22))
 (segment (start 163.4 83.82) (end 167.64 83.82) (width 0.25) (layer "F.Cu") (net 23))
 (segment (start 167.64 83.82) (end 168.91 82.55) (width 0.25) (layer "F.Cu") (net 23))
 (segment (start 168.91 82.55) (end 170.61 82.55) (width 0.25) (layer "F.Cu") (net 23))
 (segment (start 163.4 82.55) (end 167.64 82.55) (width 0.25) (layer "F.Cu") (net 24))
 (segment (start 168.91 81.28) (end 170.61 81.28) (width 0.25) (layer "F.Cu") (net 24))
 (segment (start 167.64 82.55) (end 168.91 81.28) (width 0.25) (layer "F.Cu") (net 24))
 (segment (start 167.64 81.28) (end 168.91 80.01) (width 0.25) (layer "F.Cu") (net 25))
 (segment (start 163.4 81.28) (end 167.64 81.28) (width 0.25) (layer "F.Cu") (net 25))
 (segment (start 168.91 80.01) (end 170.61 80.01) (width 0.25) (layer "F.Cu") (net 25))
 (segment (start 168.91 78.74) (end 170.61 78.74) (width 0.25) (layer "F.Cu") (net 26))
 (segment (start 167.64 80.01) (end 168.91 78.74) (width 0.25) (layer "F.Cu") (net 26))
 (segment (start 163.4 80.01) (end 167.64 80.01) (width 0.25) (layer "F.Cu") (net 26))
 (segment (start 195.469 88.789) (end 194.31 87.63) (width 0.25) (layer "F.Cu") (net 11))
 (segment (start 182.88 85.09) (end 181.61 83.82) (width 0.25) (layer "F.Cu") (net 11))
 (segment (start 194.31 87.63) (end 183.515 87.63) (width 0.25) (layer "F.Cu") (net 11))
 (segment (start 181.61 83.82) (end 179.91 83.82) (width 0.25) (layer "F.Cu") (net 11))
 (segment (start 182.88 86.995) (end 182.88 85.09) (width 0.25) (layer "F.Cu") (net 11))
 (segment (start 195.469 89.535) (end 195.469 88.789) (width 0.25) (layer "F.Cu") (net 11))
 (segment (start 183.515 87.63) (end 182.88 86.995) (width 0.25) (layer "F.Cu") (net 11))
 (segment (start 183.515 84.455) (end 185.4725 84.455) (width 0.25) (layer "F.Cu") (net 3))
 (segment (start 181.61 82.55) (end 183.515 84.455) (width 0.25) (layer "F.Cu") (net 3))
 (segment (start 179.91 82.55) (end 181.61 82.55) (width 0.25) (layer "F.Cu") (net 3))
 (segment (start 181.61 81.28) (end 183.515 83.185) (width 0.25) (layer "F.Cu") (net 4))
 (segment (start 194.185 83.155) (end 195.485 84.455) (width 0.25) (layer "F.Cu") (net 4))
 (segment (start 183.545 83.155) (end 194.185 83.155) (width 0.25) (layer "F.Cu") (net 4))
 (segment (start 179.91 81.28) (end 181.61 81.28) (width 0.25) (layer "F.Cu") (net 4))
 (segment (start 183.515 83.185) (end 183.545 83.155) (width 0.25) (layer "F.Cu") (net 4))
 (segment (start 182.88 80.01) (end 183.545 80.675) (width 0.25) (layer "F.Cu") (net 31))
 (segment (start 179.91 80.01) (end 182.88 80.01) (width 0.25) (layer "F.Cu") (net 31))
 (segment (start 183.545 80.675) (end 194.28 80.675) (width 0.25) (layer "F.Cu") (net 31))
 (segment (start 194.28 80.675) (end 195.485 79.47) (width 0.25) (layer "F.Cu") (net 31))
 (segment (start 195.485 79.47) (end 195.485 79.375) (width 0.25) (layer "F.Cu") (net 31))
 (segment (start 179.91 78.74) (end 182.245 78.74) (width 0.25) (layer "F.Cu") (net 32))
 (segment (start 182.88 79.375) (end 185.4725 79.375) (width 0.25) (layer "F.Cu") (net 32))
 (segment (start 182.245 78.74) (end 182.88 79.375) (width 0.25) (layer "F.Cu") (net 32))
 (segment (start 179.91 77.47) (end 182.88 77.47) (width 0.25) (layer "F.Cu") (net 8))
 (segment (start 194.185 76.23) (end 195.485 74.93) (width 0.25) (layer "F.Cu") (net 8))
 (segment (start 184.18 76.23) (end 194.185 76.23) (width 0.25) (layer "F.Cu") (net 8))
 (segment (start 184.15 76.2) (end 184.18 76.23) (width 0.25) (layer "F.Cu") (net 8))
 (segment (start 182.88 77.47) (end 184.15 76.2) (width 0.25) (layer "F.Cu") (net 8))
 (segment (start 179.91 76.2) (end 181.18 74.93) (width 0.25) (layer "F.Cu") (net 33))
 (segment (start 181.18 74.93) (end 185.4725 74.93) (width 0.25) (layer "F.Cu") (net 33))
 (segment (start 167.64 78.74) (end 168.91 77.47) (width 0.25) (layer "F.Cu") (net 27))
 (segment (start 168.91 77.47) (end 170.61 77.47) (width 0.25) (layer "F.Cu") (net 27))
 (segment (start 163.4 78.74) (end 167.64 78.74) (width 0.25) (layer "F.Cu") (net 27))
 (segment (start 163.4 77.47) (end 167.64 77.47) (width 0.25) (layer "F.Cu") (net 28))
 (segment (start 168.91 76.2) (end 170.61 76.2) (width 0.25) (layer "F.Cu") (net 28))
 (segment (start 167.64 77.47) (end 168.91 76.2) (width 0.25) (layer "F.Cu") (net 28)))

